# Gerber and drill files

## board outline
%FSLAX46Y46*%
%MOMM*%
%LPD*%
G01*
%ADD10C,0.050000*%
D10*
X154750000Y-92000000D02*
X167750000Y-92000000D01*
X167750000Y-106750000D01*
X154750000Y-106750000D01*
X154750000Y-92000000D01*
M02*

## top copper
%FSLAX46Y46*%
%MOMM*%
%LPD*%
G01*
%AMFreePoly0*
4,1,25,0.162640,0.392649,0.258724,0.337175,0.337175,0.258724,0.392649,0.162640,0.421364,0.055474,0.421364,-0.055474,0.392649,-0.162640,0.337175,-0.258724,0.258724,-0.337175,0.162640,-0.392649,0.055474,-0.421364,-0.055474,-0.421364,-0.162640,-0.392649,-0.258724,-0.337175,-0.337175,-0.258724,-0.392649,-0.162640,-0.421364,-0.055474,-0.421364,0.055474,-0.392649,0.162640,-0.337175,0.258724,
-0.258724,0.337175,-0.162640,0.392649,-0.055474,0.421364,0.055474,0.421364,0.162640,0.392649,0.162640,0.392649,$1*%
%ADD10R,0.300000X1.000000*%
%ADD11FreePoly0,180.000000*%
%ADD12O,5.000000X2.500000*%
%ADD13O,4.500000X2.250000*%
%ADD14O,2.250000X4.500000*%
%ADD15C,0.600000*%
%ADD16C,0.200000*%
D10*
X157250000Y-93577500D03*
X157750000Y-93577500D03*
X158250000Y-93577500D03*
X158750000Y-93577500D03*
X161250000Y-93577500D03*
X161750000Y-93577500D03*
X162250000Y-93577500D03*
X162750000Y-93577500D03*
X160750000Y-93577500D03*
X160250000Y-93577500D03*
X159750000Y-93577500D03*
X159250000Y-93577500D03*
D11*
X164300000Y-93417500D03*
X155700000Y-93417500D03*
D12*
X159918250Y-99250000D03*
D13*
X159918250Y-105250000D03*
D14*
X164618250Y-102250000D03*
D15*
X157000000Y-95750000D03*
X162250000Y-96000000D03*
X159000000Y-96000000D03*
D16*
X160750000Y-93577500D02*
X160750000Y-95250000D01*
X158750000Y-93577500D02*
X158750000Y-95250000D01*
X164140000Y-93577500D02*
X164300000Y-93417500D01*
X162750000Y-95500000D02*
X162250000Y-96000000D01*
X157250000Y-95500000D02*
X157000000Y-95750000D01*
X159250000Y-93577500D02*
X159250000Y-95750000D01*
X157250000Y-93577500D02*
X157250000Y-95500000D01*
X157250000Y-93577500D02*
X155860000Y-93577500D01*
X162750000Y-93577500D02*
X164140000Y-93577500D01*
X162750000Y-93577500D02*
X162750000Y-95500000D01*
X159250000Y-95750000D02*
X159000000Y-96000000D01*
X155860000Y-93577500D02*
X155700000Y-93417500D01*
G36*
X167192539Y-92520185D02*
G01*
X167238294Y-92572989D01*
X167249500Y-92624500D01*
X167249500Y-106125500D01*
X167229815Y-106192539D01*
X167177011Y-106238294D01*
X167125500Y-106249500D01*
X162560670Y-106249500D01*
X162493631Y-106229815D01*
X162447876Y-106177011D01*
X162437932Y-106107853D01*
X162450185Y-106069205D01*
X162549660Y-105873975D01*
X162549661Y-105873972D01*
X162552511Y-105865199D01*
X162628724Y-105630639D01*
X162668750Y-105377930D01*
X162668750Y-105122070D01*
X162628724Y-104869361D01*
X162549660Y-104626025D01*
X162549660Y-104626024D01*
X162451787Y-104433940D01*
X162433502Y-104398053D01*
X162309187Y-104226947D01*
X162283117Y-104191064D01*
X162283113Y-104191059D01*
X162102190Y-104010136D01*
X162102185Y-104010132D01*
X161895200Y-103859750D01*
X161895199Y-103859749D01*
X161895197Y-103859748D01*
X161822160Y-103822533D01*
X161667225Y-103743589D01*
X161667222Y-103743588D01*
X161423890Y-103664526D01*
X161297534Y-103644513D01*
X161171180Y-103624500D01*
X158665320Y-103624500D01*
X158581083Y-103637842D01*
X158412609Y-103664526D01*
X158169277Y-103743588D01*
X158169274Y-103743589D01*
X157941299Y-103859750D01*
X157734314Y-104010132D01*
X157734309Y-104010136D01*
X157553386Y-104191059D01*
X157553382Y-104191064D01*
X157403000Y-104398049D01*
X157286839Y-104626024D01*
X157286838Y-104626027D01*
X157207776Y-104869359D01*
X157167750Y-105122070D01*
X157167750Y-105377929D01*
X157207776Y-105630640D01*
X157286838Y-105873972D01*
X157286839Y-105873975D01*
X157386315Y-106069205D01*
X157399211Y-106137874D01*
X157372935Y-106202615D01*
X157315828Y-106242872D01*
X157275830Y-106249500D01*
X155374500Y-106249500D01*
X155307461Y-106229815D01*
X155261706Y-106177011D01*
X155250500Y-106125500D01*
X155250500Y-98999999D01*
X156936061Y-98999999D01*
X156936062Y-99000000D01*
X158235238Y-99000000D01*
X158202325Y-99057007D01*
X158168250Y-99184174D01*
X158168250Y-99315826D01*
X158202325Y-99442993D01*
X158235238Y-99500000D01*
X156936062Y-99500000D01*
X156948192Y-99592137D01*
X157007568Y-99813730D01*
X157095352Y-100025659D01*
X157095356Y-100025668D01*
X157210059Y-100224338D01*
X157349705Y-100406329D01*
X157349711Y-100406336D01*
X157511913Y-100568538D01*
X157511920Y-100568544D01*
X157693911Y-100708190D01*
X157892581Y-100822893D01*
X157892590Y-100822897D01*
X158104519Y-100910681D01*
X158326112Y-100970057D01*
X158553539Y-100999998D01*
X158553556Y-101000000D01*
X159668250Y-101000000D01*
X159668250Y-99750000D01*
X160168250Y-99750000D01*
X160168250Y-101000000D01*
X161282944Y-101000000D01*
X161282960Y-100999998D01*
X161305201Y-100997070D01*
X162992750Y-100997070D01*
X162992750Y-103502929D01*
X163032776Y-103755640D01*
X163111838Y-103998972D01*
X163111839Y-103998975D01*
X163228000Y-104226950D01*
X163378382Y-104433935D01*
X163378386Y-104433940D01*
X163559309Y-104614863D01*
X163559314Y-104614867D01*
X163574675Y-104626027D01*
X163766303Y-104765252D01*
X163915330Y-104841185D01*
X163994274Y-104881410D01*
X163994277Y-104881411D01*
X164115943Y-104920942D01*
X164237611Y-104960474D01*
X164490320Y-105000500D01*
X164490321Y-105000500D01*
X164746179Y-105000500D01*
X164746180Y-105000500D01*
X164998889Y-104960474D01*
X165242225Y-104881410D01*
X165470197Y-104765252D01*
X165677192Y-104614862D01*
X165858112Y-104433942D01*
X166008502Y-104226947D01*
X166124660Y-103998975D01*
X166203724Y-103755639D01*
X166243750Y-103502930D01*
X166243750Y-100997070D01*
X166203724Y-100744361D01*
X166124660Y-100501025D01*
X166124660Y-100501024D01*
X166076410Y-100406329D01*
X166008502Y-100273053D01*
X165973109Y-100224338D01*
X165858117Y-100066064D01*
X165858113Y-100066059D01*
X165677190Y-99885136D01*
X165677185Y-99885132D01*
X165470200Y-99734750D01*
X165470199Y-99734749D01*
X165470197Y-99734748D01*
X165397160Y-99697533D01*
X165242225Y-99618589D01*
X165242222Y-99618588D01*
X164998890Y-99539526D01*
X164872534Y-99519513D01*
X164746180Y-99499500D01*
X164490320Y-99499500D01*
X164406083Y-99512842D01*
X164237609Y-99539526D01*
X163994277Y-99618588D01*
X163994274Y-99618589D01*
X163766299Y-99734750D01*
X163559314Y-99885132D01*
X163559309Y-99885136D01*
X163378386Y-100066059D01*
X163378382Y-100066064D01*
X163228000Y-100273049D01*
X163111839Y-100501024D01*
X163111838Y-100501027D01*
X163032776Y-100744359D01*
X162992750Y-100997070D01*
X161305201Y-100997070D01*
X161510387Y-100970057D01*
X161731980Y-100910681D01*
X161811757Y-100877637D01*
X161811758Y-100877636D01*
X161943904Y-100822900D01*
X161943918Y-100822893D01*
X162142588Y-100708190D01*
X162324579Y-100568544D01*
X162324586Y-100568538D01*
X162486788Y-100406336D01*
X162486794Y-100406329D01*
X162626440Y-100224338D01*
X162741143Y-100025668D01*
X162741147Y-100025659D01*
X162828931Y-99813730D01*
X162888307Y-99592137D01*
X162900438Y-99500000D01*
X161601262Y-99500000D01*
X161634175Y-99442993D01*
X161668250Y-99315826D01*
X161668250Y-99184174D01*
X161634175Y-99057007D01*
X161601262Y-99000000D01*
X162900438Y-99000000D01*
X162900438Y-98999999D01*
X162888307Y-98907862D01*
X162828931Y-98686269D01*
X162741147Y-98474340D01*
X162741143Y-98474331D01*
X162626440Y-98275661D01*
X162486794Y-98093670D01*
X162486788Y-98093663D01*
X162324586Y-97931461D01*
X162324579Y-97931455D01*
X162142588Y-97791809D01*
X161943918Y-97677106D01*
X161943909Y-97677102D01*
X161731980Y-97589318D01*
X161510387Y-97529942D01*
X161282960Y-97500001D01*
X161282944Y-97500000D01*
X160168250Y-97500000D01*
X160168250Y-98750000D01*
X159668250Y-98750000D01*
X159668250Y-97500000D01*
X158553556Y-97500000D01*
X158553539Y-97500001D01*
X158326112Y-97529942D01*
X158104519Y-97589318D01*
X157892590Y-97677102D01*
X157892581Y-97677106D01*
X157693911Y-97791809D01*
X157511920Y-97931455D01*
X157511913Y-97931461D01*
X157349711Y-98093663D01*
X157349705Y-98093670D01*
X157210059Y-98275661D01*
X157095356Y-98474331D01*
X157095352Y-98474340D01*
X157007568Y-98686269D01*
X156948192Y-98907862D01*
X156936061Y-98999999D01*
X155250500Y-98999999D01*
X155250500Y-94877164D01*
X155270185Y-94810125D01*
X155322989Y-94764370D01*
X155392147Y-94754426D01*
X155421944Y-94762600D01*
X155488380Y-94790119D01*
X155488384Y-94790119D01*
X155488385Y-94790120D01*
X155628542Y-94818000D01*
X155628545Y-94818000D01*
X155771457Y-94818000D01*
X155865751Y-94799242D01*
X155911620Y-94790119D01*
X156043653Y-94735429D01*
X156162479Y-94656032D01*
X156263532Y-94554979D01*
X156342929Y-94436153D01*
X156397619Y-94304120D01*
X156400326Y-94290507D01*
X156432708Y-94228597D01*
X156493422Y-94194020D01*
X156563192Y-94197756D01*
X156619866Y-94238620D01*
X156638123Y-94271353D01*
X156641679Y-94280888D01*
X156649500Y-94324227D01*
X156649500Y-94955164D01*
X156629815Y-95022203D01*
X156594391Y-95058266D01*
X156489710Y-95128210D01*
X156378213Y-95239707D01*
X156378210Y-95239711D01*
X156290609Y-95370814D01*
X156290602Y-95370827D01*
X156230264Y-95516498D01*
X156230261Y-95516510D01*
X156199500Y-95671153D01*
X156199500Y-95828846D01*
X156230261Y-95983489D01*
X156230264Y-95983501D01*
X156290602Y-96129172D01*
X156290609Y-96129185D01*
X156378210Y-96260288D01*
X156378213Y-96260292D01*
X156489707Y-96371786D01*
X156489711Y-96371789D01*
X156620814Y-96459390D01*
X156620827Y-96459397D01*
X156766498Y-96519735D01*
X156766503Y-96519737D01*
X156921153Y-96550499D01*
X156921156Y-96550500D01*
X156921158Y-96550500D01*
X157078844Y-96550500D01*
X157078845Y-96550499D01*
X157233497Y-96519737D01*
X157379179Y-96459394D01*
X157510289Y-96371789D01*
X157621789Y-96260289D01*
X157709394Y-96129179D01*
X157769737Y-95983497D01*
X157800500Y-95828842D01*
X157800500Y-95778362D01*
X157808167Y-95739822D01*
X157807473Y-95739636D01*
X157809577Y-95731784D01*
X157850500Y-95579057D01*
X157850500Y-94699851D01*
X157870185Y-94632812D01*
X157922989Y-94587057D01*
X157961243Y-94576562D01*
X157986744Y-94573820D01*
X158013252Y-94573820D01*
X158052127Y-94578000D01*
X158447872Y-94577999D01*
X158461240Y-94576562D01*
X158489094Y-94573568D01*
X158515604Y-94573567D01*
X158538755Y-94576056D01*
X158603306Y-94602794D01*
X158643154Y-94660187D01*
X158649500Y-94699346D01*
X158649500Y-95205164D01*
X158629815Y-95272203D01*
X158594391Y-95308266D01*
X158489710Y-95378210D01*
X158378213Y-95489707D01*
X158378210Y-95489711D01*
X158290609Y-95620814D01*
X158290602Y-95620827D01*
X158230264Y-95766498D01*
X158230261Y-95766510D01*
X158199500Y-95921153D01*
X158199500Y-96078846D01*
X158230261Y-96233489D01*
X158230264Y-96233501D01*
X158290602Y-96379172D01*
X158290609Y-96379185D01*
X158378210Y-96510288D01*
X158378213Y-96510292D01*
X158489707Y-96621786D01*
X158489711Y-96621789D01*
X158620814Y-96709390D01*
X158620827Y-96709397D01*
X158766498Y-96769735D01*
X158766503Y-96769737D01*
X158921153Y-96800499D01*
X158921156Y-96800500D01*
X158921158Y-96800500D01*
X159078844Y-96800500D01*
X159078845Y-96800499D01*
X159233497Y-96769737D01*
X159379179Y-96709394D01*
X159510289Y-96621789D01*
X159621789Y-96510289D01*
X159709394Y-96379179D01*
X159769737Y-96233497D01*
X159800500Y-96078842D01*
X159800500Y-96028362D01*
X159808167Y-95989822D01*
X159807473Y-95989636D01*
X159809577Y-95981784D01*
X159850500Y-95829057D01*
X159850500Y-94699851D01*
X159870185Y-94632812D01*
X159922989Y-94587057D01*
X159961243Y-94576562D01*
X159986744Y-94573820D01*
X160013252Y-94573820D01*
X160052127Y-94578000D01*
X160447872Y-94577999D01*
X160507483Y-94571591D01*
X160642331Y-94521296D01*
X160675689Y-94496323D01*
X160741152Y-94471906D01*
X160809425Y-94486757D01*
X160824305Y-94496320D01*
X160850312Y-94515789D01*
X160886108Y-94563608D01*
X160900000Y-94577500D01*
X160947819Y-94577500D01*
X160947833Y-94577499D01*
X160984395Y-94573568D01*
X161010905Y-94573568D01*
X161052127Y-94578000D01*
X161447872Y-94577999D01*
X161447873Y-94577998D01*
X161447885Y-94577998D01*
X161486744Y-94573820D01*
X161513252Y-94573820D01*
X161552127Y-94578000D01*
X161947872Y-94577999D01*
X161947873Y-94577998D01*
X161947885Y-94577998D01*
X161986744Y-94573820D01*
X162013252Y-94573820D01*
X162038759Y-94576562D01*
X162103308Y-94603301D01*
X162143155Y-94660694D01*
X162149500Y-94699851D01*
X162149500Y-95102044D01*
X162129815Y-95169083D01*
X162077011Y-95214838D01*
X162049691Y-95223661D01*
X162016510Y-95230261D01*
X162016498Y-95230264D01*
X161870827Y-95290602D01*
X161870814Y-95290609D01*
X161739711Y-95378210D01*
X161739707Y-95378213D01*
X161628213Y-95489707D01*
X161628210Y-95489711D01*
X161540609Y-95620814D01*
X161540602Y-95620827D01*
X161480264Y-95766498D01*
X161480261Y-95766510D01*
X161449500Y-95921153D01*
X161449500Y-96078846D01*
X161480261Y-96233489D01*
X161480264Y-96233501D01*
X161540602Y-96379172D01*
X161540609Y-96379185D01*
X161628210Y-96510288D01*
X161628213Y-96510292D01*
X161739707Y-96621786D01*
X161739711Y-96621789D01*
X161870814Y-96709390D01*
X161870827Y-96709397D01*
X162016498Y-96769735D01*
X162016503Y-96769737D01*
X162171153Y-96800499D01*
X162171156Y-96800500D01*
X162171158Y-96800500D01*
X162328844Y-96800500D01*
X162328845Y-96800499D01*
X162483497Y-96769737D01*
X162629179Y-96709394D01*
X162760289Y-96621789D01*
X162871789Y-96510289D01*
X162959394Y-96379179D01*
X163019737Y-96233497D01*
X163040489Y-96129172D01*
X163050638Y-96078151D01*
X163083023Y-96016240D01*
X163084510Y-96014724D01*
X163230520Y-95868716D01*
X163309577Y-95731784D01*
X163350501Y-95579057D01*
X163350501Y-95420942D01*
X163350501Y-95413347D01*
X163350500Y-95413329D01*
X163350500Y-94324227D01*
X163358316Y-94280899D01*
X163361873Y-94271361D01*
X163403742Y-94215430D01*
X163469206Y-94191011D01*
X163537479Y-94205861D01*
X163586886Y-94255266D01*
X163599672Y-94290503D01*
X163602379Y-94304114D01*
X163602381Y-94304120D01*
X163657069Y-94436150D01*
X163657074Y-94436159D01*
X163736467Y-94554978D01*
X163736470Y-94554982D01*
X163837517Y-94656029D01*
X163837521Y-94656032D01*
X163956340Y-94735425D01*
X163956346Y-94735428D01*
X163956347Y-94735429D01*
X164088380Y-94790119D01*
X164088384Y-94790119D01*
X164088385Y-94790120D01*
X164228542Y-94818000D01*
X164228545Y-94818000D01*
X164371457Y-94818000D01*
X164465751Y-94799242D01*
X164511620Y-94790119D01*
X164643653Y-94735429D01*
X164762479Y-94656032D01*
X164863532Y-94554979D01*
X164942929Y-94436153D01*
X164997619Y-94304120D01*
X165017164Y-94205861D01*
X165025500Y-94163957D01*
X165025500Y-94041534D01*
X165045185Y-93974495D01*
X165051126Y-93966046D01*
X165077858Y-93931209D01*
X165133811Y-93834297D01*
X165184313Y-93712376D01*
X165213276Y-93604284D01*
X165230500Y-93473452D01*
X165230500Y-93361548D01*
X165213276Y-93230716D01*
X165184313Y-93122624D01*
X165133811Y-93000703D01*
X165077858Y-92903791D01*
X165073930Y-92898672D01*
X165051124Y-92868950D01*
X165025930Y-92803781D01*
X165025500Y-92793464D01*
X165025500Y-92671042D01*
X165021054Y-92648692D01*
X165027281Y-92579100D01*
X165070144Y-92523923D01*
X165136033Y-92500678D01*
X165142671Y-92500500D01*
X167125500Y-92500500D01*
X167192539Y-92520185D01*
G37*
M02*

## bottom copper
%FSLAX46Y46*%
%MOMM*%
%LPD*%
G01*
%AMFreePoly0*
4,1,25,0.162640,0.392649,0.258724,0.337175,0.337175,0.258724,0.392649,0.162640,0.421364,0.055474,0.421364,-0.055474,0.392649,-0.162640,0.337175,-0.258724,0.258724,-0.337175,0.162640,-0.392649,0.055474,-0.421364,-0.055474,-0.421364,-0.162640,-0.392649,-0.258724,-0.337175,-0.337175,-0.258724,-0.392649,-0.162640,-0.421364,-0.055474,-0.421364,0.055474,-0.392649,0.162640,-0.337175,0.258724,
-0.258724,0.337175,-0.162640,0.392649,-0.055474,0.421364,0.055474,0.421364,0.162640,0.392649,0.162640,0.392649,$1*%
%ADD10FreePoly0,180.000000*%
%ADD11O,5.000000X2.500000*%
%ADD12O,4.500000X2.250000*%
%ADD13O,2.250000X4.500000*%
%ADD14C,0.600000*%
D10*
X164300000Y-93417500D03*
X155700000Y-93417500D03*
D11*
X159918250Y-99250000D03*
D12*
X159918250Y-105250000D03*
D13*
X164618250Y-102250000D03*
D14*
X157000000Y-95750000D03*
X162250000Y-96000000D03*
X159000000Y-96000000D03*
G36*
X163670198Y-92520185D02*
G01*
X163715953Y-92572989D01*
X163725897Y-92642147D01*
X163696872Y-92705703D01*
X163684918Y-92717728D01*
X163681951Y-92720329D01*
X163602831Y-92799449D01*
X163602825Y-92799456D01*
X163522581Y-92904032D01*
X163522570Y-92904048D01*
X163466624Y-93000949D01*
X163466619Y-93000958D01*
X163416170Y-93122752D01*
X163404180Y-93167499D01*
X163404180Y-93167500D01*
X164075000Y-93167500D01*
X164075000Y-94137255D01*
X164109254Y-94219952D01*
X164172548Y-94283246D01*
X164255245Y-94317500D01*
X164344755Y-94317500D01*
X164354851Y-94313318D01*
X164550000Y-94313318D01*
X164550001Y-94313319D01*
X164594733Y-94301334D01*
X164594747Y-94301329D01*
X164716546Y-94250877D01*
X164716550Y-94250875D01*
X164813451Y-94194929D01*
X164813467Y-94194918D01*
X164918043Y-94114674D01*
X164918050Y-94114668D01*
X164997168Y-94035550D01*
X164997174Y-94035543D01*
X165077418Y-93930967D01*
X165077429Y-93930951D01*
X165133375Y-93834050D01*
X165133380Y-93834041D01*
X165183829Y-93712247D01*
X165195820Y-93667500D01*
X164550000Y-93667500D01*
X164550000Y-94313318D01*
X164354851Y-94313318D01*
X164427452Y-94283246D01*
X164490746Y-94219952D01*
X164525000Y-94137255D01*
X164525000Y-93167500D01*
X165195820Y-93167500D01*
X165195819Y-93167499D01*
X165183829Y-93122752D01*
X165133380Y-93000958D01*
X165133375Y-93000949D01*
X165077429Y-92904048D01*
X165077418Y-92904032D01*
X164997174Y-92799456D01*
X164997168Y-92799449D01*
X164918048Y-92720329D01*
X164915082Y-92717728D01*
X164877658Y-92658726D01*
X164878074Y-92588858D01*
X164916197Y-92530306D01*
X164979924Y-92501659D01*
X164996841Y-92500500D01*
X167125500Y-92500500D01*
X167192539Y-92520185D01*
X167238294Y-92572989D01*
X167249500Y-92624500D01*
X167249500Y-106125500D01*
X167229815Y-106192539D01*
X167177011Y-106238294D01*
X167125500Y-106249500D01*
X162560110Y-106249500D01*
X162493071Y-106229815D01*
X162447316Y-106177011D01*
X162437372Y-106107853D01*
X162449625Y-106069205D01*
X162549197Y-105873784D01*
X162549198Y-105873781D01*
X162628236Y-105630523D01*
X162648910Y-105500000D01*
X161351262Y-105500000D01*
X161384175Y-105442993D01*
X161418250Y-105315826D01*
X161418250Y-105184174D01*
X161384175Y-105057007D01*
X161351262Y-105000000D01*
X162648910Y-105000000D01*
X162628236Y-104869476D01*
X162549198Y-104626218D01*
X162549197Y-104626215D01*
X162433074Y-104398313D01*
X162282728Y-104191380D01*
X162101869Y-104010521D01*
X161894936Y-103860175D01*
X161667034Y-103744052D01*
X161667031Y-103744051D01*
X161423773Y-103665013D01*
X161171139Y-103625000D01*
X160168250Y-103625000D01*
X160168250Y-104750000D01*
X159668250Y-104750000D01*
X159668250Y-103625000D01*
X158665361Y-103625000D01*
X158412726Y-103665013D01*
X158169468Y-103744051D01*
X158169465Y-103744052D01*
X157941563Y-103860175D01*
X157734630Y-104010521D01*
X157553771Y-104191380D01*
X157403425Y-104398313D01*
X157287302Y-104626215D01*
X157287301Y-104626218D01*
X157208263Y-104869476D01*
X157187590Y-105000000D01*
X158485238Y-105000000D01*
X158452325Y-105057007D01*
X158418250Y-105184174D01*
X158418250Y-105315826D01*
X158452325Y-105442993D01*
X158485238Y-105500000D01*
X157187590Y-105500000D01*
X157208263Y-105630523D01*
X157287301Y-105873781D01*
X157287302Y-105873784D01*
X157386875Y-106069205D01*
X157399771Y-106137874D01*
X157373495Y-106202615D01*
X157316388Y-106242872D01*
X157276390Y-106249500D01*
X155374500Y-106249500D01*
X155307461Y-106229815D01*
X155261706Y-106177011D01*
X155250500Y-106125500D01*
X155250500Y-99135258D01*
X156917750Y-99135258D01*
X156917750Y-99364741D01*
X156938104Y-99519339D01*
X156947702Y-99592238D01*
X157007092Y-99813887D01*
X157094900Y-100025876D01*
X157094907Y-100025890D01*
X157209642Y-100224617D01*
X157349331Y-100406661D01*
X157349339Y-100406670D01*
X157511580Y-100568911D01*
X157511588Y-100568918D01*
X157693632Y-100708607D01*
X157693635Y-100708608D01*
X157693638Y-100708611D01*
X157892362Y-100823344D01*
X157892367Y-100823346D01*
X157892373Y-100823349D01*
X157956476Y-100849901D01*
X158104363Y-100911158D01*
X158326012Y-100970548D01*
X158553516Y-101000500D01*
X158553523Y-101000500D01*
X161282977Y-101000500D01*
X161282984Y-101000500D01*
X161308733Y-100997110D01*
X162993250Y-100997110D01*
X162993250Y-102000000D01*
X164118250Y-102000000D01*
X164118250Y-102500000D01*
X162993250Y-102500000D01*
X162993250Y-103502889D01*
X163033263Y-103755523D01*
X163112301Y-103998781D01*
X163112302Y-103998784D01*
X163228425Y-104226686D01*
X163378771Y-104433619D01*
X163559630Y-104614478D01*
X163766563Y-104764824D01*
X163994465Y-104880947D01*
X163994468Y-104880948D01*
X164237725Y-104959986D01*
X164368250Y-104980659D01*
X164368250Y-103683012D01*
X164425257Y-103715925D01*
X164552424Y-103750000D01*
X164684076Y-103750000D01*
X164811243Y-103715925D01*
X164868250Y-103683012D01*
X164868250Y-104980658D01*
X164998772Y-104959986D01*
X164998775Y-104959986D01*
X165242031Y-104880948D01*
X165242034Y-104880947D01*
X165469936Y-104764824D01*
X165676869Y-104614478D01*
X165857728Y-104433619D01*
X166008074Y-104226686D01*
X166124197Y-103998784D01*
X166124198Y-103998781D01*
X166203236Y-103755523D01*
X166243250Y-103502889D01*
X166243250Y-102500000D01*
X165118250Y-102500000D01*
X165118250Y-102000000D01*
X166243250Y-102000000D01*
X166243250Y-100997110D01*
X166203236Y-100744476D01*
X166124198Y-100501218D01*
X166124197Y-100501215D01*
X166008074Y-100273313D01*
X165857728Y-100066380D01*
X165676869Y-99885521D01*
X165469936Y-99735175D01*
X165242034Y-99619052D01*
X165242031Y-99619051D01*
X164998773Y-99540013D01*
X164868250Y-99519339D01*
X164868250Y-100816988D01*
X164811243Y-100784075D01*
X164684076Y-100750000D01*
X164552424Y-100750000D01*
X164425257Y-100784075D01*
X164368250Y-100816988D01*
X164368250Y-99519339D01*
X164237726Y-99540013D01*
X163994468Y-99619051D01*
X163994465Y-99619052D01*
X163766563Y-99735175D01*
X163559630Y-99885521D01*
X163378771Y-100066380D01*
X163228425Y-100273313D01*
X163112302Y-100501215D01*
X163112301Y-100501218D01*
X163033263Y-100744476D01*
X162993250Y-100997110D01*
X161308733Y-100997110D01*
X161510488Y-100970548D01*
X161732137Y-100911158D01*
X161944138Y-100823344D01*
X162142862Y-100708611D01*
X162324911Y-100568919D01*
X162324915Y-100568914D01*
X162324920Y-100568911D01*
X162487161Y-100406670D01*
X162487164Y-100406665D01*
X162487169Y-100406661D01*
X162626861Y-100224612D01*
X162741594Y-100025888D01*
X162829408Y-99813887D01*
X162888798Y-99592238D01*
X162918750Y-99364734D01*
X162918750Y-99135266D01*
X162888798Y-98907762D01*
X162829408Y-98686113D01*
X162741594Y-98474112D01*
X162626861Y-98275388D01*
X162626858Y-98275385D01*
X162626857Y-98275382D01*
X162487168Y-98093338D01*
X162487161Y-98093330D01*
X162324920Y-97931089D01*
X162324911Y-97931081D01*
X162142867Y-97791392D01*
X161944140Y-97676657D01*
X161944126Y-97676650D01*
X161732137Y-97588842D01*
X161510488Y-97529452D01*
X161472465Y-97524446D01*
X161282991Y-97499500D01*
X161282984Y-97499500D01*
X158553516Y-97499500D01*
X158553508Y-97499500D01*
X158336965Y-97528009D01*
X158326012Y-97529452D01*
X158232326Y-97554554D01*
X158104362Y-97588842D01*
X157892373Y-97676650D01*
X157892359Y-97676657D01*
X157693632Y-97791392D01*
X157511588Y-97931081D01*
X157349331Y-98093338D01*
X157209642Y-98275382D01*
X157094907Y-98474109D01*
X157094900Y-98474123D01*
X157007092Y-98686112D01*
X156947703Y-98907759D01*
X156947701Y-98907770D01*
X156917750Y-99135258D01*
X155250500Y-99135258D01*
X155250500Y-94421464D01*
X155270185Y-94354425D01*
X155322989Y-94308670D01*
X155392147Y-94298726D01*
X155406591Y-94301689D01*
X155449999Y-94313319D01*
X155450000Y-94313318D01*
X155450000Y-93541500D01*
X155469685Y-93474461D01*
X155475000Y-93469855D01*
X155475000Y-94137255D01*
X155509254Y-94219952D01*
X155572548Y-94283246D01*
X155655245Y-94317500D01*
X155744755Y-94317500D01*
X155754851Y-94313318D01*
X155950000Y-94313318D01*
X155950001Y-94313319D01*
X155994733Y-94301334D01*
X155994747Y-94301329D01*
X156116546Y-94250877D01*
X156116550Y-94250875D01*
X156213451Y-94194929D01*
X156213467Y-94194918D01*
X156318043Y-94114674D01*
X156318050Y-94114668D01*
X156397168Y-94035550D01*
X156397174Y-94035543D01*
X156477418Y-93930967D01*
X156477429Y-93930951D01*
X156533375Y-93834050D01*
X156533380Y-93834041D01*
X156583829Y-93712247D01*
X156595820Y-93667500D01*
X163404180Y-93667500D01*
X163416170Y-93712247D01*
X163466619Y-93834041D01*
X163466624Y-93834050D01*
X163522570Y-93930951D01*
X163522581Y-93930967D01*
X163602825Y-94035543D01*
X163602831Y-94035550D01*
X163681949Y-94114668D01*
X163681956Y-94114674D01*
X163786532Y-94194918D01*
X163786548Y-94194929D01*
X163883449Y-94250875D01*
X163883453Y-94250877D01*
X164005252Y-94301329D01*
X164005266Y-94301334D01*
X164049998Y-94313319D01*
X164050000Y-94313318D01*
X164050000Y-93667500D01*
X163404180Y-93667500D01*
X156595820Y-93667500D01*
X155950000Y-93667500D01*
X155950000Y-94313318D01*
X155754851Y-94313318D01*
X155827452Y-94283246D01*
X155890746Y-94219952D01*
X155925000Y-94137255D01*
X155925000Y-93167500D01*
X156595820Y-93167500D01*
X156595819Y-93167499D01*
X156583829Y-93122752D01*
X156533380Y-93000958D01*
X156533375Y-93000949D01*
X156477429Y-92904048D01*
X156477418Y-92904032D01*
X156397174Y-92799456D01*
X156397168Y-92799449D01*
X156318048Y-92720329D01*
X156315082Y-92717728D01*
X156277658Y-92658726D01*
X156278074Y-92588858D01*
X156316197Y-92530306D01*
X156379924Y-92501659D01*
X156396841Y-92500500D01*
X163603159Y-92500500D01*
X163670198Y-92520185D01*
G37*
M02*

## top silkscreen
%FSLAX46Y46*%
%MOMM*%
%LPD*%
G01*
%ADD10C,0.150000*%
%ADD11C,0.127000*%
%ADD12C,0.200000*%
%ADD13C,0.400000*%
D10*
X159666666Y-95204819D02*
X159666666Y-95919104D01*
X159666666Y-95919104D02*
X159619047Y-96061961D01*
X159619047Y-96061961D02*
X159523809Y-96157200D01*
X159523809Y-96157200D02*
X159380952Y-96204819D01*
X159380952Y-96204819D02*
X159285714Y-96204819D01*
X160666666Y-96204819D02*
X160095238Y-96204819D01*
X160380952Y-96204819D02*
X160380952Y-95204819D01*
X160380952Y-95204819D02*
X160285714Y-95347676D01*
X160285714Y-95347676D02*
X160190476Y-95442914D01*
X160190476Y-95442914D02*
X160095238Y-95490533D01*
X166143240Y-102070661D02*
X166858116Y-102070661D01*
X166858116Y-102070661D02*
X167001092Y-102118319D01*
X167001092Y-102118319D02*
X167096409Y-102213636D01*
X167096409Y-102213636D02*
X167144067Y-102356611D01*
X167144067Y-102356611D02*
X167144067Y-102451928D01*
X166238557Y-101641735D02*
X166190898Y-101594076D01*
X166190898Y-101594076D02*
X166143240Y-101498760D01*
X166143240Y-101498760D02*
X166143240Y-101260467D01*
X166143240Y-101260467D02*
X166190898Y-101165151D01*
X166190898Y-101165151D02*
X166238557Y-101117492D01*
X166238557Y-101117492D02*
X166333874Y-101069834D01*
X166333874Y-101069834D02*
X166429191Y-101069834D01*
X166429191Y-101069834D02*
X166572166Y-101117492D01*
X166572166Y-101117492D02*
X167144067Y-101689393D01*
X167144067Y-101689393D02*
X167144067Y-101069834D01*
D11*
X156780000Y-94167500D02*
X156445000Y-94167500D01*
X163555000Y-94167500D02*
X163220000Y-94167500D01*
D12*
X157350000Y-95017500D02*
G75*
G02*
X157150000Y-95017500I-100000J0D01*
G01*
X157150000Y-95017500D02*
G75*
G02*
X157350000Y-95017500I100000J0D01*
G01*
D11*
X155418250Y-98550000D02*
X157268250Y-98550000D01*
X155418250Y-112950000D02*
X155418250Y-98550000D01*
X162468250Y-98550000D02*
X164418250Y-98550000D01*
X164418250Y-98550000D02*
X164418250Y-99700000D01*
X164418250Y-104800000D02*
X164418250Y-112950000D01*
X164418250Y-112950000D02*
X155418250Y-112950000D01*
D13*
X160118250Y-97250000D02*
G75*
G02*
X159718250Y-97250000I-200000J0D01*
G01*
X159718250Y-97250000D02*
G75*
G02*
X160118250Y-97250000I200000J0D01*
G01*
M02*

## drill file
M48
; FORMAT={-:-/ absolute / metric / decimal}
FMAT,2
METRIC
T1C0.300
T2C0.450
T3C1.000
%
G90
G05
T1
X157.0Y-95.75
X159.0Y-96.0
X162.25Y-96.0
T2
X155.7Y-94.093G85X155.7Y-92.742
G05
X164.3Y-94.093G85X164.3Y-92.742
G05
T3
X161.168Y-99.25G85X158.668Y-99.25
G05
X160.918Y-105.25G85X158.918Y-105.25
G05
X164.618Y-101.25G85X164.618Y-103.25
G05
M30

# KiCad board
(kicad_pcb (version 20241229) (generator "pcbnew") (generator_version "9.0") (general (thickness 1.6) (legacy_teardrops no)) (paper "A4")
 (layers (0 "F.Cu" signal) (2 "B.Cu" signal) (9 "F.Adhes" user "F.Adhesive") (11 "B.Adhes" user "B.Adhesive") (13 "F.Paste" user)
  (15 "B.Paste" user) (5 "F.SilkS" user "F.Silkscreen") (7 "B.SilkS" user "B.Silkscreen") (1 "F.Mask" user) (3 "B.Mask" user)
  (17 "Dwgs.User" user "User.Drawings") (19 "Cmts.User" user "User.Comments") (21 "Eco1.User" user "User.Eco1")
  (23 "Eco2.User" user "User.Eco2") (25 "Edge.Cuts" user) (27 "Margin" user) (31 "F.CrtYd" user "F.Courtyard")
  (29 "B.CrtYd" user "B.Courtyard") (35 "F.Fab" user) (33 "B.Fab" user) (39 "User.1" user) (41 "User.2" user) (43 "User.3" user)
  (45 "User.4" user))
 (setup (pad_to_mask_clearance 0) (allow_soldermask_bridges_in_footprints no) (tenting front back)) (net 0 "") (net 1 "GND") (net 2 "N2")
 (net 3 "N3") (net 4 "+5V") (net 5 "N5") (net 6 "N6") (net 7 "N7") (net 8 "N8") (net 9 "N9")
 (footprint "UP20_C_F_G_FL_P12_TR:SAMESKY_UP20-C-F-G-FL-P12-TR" (layer "F.Cu") (at 160 92.0175 180)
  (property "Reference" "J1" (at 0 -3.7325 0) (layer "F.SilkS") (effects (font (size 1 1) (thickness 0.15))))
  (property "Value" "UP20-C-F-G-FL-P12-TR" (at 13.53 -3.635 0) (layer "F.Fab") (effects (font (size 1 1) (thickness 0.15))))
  (fp_line (start 3.22 -2.15) (end 3.555 -2.15) (stroke (width 0.127) (type solid)) (layer "F.SilkS"))
  (fp_line (start -3.555 -2.15) (end -3.22 -2.15) (stroke (width 0.127) (type solid)) (layer "F.SilkS"))
  (fp_circle (center 2.75 -3) (end 2.85 -3) (stroke (width 0.2) (type solid)) (fill no) (layer "F.SilkS"))
  (pad "A1" smd rect (at 2.75 -1.56 180) (size 0.3 1) (layers "F.Cu" "F.Mask" "F.Paste") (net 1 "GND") (solder_mask_margin 0.102))
  (pad "A2" smd rect (at 2.25 -1.56 180) (size 0.3 1) (layers "F.Cu" "F.Mask" "F.Paste") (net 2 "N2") (solder_mask_margin 0.102))
  (pad "A3" smd rect (at 1.75 -1.56 180) (size 0.3 1) (layers "F.Cu" "F.Mask" "F.Paste") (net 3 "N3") (solder_mask_margin 0.102))
  (pad "A4" smd rect (at 1.25 -1.56 180) (size 0.3 1) (layers "F.Cu" "F.Mask" "F.Paste") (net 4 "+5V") (solder_mask_margin 0.102))
  (pad "A5" smd rect (at -1.25 -1.56 180) (size 0.3 1) (layers "F.Cu" "F.Mask" "F.Paste") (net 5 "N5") (solder_mask_margin 0.102))
  (pad "A6" smd rect (at -1.75 -1.56 180) (size 0.3 1) (layers "F.Cu" "F.Mask" "F.Paste") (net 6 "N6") (solder_mask_margin 0.102))
  (pad "A7" smd rect (at -2.25 -1.56 180) (size 0.3 1) (layers "F.Cu" "F.Mask" "F.Paste") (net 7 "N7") (solder_mask_margin 0.102))
  (pad "A12" smd rect (at -2.75 -1.56 180) (size 0.3 1) (layers "F.Cu" "F.Mask" "F.Paste") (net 1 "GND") (solder_mask_margin 0.102))
  (pad "B9" smd rect (at -0.75 -1.56 180) (size 0.3 1) (layers "F.Cu" "F.Mask" "F.Paste") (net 4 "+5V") (solder_mask_margin 0.102))
  (pad "B10" smd rect (at -0.25 -1.56 180) (size 0.3 1) (layers "F.Cu" "F.Mask" "F.Paste") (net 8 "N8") (solder_mask_margin 0.102))
  (pad "B11" smd rect (at 0.25 -1.56 180) (size 0.3 1) (layers "F.Cu" "F.Mask" "F.Paste") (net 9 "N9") (solder_mask_margin 0.102))
  (pad "B12" smd rect (at 0.75 -1.56 180) (size 0.3 1) (layers "F.Cu" "F.Mask" "F.Paste") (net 1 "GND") (solder_mask_margin 0.102))
  (pad "SH1" thru_hole custom (at -4.3 -1.4 180) (size 0.85 2.25) (drill oval 0.45 1.8) (layers "*.Cu") (remove_unused_layers no)
   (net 1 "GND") (thermal_bridge_angle 90) (options (clearance outline) (anchor circle)) (primitives))
  (pad "SH2" thru_hole custom (at 4.3 -1.4 180) (size 0.85 2.25) (drill oval 0.45 1.8) (layers "*.Cu") (remove_unused_layers no)
   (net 1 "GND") (thermal_bridge_angle 90) (options (clearance outline) (anchor circle)) (primitives)))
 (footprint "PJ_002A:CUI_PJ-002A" (layer "F.Cu") (at 159.91825 99.25 -90)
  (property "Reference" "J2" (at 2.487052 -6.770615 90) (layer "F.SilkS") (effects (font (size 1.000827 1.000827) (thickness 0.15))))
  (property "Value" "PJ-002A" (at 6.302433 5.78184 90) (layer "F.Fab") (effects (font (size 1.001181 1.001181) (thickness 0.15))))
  (fp_line (start -0.7 4.5) (end -0.7 2.65) (stroke (width 0.127) (type solid)) (layer "F.SilkS"))
  (fp_line (start 13.7 4.5) (end -0.7 4.5) (stroke (width 0.127) (type solid)) (layer "F.SilkS"))
  (fp_line (start -0.7 -2.55) (end -0.7 -4.5) (stroke (width 0.127) (type solid)) (layer "F.SilkS"))
  (fp_line (start -0.7 -4.5) (end 0.45 -4.5) (stroke (width 0.127) (type solid)) (layer "F.SilkS"))
  (fp_line (start 5.55 -4.5) (end 13.7 -4.5) (stroke (width 0.127) (type solid)) (layer "F.SilkS"))
  (fp_line (start 13.7 -4.5) (end 13.7 4.5) (stroke (width 0.127) (type solid)) (layer "F.SilkS"))
  (fp_circle (center -2 0) (end -1.8 0) (stroke (width 0.4) (type solid)) (fill no) (layer "F.SilkS"))
  (pad "1" thru_hole oval (at 0 0 270) (size 2.5 5) (drill oval 1 3.5) (layers "*.Cu" "*.Mask") (remove_unused_layers no) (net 4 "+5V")
   (solder_mask_margin 0.102))
  (pad "2" thru_hole oval (at 6 0 270) (size 2.25 4.5) (drill oval 1 3) (layers "*.Cu" "*.Mask") (remove_unused_layers no) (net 1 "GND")
   (solder_mask_margin 0.102))
  (pad "3" thru_hole oval (at 3 -4.7 270) (size 4.5 2.25) (drill oval 3 1) (layers "*.Cu" "*.Mask") (remove_unused_layers no) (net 1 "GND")
   (solder_mask_margin 0.102)))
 (gr_rect (start 154.75 92) (end 167.75 106.75) (stroke (width 0.05) (type default)) (fill no) (layer "Edge.Cuts"))
 (segment (start 160.75 93.5775) (end 160.75 95.25) (width 0.2) (layer "F.Cu") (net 4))
 (segment (start 158.75 93.5775) (end 158.75 95.25) (width 0.2) (layer "F.Cu") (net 4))
 (segment (start 164.14 93.5775) (end 164.3 93.4175) (width 0.2) (layer "F.Cu") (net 1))
 (segment (start 162.75 95.5) (end 162.25 96) (width 0.2) (layer "F.Cu") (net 1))
 (segment (start 157.25 95.5) (end 157 95.75) (width 0.2) (layer "F.Cu") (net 1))
 (segment (start 159.25 93.5775) (end 159.25 95.75) (width 0.2) (layer "F.Cu") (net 1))
 (segment (start 157.25 93.5775) (end 157.25 95.5) (width 0.2) (layer "F.Cu") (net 1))
 (segment (start 157.25 93.5775) (end 155.86 93.5775) (width 0.2) (layer "F.Cu") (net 1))
 (segment (start 162.75 93.5775) (end 164.14 93.5775) (width 0.2) (layer "F.Cu") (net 1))
 (segment (start 162.75 93.5775) (end 162.75 95.5) (width 0.2) (layer "F.Cu") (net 1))
 (segment (start 159.25 95.75) (end 159 96) (width 0.2) (layer "F.Cu") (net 1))
 (segment (start 155.86 93.5775) (end 155.7 93.4175) (width 0.2) (layer "F.Cu") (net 1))
 (via (at 157 95.75) (size 0.6) (drill 0.3) (layers "F.Cu" "B.Cu") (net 1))
 (via (at 162.25 96) (size 0.6) (drill 0.3) (layers "F.Cu" "B.Cu") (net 1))
 (via (at 159 96) (size 0.6) (drill 0.3) (layers "F.Cu" "B.Cu") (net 1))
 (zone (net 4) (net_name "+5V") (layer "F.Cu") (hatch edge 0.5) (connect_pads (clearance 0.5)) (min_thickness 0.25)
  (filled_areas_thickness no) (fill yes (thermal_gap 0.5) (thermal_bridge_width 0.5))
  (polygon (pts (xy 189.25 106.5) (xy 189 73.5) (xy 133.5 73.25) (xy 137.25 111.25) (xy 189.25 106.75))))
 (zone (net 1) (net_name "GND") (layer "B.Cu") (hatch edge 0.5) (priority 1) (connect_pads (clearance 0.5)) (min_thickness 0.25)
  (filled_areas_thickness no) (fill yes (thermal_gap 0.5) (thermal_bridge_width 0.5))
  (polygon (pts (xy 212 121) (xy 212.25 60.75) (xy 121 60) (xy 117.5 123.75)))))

